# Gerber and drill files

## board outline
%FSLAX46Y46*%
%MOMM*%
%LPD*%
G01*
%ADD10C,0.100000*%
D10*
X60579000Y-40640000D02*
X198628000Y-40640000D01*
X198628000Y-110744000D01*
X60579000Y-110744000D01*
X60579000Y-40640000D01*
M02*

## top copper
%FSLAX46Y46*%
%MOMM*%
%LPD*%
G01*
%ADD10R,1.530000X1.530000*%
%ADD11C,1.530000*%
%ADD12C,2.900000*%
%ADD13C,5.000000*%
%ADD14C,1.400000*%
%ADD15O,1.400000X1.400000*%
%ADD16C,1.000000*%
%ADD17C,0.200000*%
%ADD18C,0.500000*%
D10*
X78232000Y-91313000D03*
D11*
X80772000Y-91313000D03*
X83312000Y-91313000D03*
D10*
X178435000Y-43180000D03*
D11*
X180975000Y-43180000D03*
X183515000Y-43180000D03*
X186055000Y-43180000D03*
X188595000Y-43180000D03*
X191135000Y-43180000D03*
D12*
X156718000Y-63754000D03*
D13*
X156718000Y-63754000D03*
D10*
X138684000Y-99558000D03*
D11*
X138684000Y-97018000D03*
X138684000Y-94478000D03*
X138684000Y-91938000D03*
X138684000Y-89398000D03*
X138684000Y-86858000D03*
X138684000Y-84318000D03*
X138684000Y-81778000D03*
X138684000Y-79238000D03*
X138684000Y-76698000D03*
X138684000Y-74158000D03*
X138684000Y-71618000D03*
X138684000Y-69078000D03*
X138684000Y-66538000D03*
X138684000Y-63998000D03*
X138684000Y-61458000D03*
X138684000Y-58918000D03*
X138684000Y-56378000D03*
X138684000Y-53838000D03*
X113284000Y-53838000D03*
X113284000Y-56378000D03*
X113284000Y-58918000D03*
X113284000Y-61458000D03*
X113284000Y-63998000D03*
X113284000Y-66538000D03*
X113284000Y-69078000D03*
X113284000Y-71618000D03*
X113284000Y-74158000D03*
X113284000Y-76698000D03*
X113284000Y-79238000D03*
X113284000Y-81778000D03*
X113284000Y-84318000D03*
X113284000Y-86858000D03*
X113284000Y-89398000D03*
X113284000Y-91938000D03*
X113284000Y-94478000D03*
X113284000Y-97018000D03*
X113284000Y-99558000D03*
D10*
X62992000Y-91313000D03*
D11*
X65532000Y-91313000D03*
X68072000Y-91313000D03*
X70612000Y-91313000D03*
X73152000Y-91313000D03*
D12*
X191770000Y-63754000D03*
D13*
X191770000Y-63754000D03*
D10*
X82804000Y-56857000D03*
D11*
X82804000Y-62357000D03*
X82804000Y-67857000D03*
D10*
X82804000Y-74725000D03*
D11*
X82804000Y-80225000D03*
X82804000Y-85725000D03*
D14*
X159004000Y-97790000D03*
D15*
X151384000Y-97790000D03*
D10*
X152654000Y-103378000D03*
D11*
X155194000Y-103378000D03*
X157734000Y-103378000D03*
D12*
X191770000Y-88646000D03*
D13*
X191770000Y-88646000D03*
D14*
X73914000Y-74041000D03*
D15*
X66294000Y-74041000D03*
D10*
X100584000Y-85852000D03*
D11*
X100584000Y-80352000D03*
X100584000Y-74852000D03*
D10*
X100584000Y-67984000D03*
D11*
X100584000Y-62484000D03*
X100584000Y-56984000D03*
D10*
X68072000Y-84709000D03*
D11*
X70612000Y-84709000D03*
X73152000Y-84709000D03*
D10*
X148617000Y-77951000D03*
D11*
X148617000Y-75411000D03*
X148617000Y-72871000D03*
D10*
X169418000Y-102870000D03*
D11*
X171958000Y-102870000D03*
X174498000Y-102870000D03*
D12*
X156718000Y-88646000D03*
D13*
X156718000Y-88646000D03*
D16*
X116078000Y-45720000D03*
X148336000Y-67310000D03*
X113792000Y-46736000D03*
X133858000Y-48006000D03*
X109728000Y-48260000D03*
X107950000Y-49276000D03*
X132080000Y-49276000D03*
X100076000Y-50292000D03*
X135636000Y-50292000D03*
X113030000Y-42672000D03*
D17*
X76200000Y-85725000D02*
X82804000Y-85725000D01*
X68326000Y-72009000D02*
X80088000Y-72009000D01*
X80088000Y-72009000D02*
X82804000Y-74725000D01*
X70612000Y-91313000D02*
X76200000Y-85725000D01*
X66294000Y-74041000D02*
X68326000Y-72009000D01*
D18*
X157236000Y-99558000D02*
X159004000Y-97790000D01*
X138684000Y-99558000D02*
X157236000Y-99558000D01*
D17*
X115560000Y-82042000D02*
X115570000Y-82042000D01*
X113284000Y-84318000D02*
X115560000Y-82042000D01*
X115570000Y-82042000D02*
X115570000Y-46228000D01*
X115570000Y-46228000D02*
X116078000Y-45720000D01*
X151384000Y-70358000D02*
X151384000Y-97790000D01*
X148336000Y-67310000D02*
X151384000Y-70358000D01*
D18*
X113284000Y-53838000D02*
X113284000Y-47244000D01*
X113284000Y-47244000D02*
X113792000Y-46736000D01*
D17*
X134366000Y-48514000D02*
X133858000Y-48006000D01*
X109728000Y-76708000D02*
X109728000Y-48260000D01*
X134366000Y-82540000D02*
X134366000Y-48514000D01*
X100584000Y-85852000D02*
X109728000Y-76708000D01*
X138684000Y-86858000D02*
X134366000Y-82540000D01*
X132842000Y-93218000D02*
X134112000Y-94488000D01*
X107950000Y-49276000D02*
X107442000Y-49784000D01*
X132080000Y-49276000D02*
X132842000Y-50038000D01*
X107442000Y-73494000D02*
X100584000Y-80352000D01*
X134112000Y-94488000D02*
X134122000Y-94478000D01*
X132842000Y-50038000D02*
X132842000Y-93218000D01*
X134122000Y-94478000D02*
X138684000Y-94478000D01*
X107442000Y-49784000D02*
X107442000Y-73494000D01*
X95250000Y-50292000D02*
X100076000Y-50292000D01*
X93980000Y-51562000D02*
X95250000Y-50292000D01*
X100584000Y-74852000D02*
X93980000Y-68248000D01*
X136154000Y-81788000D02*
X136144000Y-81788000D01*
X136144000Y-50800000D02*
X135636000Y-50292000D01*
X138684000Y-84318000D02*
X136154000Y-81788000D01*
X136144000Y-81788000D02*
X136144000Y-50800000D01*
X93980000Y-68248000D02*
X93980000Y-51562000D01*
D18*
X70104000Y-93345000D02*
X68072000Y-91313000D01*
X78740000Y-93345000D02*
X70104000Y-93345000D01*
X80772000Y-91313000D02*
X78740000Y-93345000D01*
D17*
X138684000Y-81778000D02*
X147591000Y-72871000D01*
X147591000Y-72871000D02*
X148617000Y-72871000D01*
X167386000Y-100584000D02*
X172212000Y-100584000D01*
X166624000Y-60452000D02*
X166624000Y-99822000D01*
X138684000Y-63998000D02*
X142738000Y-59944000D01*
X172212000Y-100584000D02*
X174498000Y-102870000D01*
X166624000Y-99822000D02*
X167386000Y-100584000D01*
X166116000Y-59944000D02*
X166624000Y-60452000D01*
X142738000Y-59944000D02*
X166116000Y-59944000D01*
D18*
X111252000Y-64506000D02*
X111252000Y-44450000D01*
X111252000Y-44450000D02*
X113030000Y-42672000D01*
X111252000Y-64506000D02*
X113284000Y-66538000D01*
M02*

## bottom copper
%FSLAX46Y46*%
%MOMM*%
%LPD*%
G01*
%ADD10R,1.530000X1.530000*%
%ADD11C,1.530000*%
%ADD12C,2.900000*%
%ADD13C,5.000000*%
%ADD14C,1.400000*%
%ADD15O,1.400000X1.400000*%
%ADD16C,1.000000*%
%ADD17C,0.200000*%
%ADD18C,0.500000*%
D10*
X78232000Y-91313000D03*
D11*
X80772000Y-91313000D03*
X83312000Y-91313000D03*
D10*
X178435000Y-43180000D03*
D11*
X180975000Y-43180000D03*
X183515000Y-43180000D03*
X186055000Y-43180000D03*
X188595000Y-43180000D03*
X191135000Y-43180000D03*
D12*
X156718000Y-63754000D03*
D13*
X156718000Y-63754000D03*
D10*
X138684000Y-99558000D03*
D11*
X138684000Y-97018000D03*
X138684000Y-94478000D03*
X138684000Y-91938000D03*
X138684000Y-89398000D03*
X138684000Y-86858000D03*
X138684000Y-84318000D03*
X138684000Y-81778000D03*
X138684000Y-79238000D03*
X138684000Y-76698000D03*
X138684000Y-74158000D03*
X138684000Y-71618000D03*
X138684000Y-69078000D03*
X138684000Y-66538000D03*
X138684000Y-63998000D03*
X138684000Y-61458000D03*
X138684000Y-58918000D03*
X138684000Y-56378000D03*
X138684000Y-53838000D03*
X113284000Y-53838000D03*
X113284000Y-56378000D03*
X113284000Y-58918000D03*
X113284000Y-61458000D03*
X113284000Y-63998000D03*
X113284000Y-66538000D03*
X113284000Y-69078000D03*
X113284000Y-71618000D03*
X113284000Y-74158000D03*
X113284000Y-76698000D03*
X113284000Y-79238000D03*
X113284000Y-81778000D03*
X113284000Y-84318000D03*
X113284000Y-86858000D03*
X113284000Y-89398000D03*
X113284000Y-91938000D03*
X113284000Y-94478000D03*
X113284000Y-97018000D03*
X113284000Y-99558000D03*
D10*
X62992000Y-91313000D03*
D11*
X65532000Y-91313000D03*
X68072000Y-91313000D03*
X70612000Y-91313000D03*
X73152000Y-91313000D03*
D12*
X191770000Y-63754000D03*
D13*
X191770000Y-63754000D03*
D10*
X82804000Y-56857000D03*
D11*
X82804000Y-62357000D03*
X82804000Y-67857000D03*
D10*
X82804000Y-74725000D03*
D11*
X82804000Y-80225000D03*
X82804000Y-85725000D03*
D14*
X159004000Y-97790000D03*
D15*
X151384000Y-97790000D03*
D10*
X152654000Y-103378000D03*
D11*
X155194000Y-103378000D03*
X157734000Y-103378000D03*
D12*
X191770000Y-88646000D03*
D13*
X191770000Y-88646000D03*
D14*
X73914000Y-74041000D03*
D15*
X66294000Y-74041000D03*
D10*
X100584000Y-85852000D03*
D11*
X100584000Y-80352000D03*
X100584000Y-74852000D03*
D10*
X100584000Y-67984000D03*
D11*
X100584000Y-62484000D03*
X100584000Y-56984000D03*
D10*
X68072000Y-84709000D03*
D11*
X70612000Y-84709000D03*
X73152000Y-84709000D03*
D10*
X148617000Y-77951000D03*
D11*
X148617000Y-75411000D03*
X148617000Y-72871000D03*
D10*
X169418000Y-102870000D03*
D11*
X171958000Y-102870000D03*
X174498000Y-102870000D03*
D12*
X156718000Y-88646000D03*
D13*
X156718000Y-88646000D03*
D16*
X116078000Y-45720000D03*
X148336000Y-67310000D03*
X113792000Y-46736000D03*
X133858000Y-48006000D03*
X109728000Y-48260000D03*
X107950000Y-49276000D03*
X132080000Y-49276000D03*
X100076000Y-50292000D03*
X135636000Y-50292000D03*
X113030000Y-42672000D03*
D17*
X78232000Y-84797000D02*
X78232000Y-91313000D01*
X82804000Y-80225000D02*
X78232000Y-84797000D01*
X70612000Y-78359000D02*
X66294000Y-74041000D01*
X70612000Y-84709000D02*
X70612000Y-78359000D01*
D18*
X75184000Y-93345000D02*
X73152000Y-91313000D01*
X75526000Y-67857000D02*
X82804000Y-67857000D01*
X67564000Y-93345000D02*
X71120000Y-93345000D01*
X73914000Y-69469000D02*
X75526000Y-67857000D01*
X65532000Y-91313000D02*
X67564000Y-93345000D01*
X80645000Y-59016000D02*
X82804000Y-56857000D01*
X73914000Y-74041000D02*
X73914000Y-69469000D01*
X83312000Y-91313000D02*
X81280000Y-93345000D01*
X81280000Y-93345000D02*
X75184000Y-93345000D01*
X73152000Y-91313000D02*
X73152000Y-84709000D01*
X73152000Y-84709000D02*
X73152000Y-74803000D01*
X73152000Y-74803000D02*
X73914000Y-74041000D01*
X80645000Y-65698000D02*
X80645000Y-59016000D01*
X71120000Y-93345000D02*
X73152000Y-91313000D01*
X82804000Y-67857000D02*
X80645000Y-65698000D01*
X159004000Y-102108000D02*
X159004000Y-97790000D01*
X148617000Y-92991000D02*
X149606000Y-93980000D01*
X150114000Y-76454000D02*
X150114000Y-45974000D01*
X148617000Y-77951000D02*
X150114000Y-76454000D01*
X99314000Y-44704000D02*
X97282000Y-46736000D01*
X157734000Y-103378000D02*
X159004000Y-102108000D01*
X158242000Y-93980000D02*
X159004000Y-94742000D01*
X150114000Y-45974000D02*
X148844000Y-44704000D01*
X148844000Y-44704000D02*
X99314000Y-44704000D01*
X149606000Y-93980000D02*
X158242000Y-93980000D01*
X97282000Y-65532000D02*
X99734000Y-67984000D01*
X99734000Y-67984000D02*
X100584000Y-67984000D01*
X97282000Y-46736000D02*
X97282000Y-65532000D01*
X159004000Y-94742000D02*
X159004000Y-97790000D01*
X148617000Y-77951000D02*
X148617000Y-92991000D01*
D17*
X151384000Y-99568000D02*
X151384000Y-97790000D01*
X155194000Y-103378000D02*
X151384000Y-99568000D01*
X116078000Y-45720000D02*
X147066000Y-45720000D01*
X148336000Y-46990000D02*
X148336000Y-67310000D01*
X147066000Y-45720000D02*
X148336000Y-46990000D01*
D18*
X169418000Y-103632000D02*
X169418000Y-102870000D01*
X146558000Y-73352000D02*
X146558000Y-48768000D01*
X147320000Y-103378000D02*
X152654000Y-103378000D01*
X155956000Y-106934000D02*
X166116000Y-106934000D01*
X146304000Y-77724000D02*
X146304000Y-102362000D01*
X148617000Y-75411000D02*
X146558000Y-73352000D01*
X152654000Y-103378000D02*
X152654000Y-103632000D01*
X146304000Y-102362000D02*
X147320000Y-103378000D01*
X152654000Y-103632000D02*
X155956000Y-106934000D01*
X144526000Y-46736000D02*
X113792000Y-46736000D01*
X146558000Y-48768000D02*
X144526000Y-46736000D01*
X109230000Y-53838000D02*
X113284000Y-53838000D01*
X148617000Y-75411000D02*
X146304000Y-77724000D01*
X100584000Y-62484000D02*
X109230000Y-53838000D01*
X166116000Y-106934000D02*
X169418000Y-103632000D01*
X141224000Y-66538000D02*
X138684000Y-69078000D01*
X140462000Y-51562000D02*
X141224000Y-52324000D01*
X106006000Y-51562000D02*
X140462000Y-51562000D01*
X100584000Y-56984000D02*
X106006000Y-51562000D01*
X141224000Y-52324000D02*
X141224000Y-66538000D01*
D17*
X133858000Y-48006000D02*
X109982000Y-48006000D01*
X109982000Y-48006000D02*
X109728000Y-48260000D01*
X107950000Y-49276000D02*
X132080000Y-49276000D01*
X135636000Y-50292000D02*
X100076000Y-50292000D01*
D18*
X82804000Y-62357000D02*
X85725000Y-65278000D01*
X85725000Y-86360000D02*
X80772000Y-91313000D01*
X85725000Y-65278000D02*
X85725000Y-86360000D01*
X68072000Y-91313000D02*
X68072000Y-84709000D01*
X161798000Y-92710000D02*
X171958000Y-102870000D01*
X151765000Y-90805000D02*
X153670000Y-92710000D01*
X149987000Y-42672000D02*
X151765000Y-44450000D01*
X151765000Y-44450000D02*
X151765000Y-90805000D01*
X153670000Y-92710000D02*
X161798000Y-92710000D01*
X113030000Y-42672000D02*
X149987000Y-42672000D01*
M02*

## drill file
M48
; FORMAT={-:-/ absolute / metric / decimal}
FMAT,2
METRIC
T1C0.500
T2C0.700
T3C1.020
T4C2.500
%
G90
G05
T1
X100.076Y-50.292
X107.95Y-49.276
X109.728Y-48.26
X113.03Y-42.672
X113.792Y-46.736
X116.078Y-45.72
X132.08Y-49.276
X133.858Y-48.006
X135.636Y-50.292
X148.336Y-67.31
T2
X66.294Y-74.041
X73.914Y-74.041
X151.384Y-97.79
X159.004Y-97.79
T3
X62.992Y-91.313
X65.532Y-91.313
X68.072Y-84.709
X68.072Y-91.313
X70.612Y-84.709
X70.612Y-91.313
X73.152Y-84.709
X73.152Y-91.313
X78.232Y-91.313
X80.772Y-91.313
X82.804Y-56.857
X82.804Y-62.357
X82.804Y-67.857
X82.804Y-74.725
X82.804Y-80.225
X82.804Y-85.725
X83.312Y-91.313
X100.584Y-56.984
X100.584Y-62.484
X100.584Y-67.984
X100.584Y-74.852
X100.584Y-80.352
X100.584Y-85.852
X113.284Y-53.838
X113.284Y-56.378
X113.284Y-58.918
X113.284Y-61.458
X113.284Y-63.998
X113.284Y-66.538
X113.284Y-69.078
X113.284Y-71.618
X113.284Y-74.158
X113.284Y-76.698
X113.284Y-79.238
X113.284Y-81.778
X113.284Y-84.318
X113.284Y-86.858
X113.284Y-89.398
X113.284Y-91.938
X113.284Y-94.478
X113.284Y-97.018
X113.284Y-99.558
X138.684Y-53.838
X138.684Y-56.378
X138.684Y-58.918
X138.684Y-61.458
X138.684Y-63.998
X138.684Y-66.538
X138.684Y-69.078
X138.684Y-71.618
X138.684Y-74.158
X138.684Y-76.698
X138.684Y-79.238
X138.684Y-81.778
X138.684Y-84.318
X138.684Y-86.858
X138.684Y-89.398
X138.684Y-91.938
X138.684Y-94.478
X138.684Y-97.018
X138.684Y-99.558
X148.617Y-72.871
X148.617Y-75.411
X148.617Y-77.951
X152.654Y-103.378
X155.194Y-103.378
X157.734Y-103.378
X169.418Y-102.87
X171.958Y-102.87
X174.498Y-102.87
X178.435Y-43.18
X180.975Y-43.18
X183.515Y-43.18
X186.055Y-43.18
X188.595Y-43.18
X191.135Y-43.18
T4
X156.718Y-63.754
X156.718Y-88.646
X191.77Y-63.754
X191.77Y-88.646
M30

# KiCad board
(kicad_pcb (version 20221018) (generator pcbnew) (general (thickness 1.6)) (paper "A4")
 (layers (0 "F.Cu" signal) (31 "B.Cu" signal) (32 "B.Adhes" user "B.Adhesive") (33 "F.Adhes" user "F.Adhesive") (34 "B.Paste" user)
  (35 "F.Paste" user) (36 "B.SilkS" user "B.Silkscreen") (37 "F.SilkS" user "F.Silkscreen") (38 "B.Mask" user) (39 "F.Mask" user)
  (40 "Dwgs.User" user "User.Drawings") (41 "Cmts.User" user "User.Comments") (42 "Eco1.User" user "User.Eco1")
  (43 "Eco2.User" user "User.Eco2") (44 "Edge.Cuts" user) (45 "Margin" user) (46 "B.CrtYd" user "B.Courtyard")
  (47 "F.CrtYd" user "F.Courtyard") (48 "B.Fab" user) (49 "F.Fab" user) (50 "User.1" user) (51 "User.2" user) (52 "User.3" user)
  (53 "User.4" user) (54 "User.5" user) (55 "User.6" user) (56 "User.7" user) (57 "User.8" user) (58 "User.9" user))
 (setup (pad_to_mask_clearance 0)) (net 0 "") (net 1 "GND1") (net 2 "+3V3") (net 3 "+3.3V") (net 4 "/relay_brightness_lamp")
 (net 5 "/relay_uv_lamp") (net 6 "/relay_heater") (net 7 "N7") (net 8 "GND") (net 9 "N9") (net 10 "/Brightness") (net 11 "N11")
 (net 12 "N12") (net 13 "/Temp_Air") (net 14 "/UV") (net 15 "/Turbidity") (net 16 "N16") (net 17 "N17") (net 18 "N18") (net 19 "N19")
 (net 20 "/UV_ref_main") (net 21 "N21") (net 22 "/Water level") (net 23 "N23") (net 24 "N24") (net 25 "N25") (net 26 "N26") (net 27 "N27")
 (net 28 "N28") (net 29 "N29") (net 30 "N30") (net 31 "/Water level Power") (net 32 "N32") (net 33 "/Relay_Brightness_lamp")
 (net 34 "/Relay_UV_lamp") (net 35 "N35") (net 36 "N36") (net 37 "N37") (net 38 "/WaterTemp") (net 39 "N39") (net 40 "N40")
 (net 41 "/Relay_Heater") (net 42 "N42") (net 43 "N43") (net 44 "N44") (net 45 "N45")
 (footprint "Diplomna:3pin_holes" (layer "F.Cu") (at 85.852 93.853)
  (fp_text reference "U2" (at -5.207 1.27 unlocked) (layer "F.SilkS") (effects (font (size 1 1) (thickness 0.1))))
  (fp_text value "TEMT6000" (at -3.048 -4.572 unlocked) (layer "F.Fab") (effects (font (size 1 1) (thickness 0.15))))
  (pad "1" thru_hole rect (at -7.62 -2.54) (size 1.53 1.53) (drill 1.02) (layers "*.Cu" "*.Mask") (solder_mask_margin 0.102))
  (pad "2" thru_hole circle (at -5.08 -2.54) (size 1.53 1.53) (drill 1.02) (layers "*.Cu" "*.Mask") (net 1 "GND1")
   (solder_mask_margin 0.102))
  (pad "3" thru_hole circle (at -2.54 -2.54) (size 1.53 1.53) (drill 1.02) (layers "*.Cu" "*.Mask") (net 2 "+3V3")
   (solder_mask_margin 0.102)))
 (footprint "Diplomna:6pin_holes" (layer "F.Cu") (at 193.675 48.895)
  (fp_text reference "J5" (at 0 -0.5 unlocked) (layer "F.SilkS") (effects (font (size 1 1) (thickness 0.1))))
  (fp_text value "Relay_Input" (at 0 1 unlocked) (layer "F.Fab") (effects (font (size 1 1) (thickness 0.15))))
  (pad "1" thru_hole rect (at -15.24 -5.715) (size 1.53 1.53) (drill 1.02) (layers "*.Cu" "*.Mask") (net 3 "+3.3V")
   (solder_mask_margin 0.102))
  (pad "2" thru_hole circle (at -12.7 -5.715) (size 1.53 1.53) (drill 1.02) (layers "*.Cu" "*.Mask") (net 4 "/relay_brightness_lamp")
   (solder_mask_margin 0.102))
  (pad "3" thru_hole circle (at -10.16 -5.715) (size 1.53 1.53) (drill 1.02) (layers "*.Cu" "*.Mask") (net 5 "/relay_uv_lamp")
   (solder_mask_margin 0.102))
  (pad "4" thru_hole circle (at -7.62 -5.715) (size 1.53 1.53) (drill 1.02) (layers "*.Cu" "*.Mask") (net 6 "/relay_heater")
   (solder_mask_margin 0.102))
  (pad "5" thru_hole circle (at -5.08 -5.715) (size 1.53 1.53) (drill 1.02) (layers "*.Cu" "*.Mask") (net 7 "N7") (solder_mask_margin 0.102))
  (pad "6" thru_hole circle (at -2.54 -5.715) (size 1.53 1.53) (drill 1.02) (layers "*.Cu" "*.Mask") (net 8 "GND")
   (solder_mask_margin 0.102)))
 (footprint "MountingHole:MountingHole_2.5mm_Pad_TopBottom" (layer "F.Cu") (at 156.718 63.754)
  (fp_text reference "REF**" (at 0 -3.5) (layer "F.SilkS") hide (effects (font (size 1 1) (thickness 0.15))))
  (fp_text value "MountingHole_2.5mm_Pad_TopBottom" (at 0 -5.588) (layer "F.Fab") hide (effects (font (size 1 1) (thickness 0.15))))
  (pad "1" thru_hole circle (at 0 0) (size 2.9 2.9) (drill 2.5) (layers "*.Cu" "*.Mask"))
  (pad "1" connect circle (at 0 0) (size 5 5) (layers "F.Cu" "F.Mask"))
  (pad "1" connect circle (at 0 0) (size 5 5) (layers "B.Cu" "B.Mask")))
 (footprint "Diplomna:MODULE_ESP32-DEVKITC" (layer "F.Cu") (at 125.984 76.708 180)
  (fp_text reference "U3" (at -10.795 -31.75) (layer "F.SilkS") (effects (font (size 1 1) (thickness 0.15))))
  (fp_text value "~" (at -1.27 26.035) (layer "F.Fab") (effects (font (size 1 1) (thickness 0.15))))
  (pad "1" thru_hole rect (at -12.7 -22.85 180) (size 1.53 1.53) (drill 1.02) (layers "*.Cu" "*.Mask") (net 3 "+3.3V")
   (solder_mask_margin 0.102))
  (pad "2" thru_hole circle (at -12.7 -20.31 180) (size 1.53 1.53) (drill 1.02) (layers "*.Cu" "*.Mask") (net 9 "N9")
   (solder_mask_margin 0.102))
  (pad "3" thru_hole circle (at -12.7 -17.77 180) (size 1.53 1.53) (drill 1.02) (layers "*.Cu" "*.Mask") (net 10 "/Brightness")
   (solder_mask_margin 0.102))
  (pad "4" thru_hole circle (at -12.7 -15.23 180) (size 1.53 1.53) (drill 1.02) (layers "*.Cu" "*.Mask") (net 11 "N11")
   (solder_mask_margin 0.102))
  (pad "5" thru_hole circle (at -12.7 -12.69 180) (size 1.53 1.53) (drill 1.02) (layers "*.Cu" "*.Mask") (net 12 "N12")
   (solder_mask_margin 0.102))
  (pad "6" thru_hole circle (at -12.7 -10.15 180) (size 1.53 1.53) (drill 1.02) (layers "*.Cu" "*.Mask") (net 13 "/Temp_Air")
   (solder_mask_margin 0.102))
  (pad "7" thru_hole circle (at -12.7 -7.61 180) (size 1.53 1.53) (drill 1.02) (layers "*.Cu" "*.Mask") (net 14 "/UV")
   (solder_mask_margin 0.102))
  (pad "8" thru_hole circle (at -12.7 -5.07 180) (size 1.53 1.53) (drill 1.02) (layers "*.Cu" "*.Mask") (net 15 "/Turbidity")
   (solder_mask_margin 0.102))
  (pad "9" thru_hole circle (at -12.7 -2.53 180) (size 1.53 1.53) (drill 1.02) (layers "*.Cu" "*.Mask") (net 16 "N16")
   (solder_mask_margin 0.102))
  (pad "10" thru_hole circle (at -12.7 0.01 180) (size 1.53 1.53) (drill 1.02) (layers "*.Cu" "*.Mask") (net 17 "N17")
   (solder_mask_margin 0.102))
  (pad "11" thru_hole circle (at -12.7 2.55 180) (size 1.53 1.53) (drill 1.02) (layers "*.Cu" "*.Mask") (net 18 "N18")
   (solder_mask_margin 0.102))
  (pad "12" thru_hole circle (at -12.7 5.09 180) (size 1.53 1.53) (drill 1.02) (layers "*.Cu" "*.Mask") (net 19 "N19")
   (solder_mask_margin 0.102))
  (pad "13" thru_hole circle (at -12.7 7.63 180) (size 1.53 1.53) (drill 1.02) (layers "*.Cu" "*.Mask") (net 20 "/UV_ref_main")
   (solder_mask_margin 0.102))
  (pad "14" thru_hole circle (at -12.7 10.17 180) (size 1.53 1.53) (drill 1.02) (layers "*.Cu" "*.Mask") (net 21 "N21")
   (solder_mask_margin 0.102))
  (pad "15" thru_hole circle (at -12.7 12.71 180) (size 1.53 1.53) (drill 1.02) (layers "*.Cu" "*.Mask") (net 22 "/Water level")
   (solder_mask_margin 0.102))
  (pad "16" thru_hole circle (at -12.7 15.25 180) (size 1.53 1.53) (drill 1.02) (layers "*.Cu" "*.Mask") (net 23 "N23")
   (solder_mask_margin 0.102))
  (pad "17" thru_hole circle (at -12.7 17.79 180) (size 1.53 1.53) (drill 1.02) (layers "*.Cu" "*.Mask") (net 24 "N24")
   (solder_mask_margin 0.102))
  (pad "18" thru_hole circle (at -12.7 20.33 180) (size 1.53 1.53) (drill 1.02) (layers "*.Cu" "*.Mask") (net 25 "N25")
   (solder_mask_margin 0.102))
  (pad "19" thru_hole circle (at -12.7 22.87 180) (size 1.53 1.53) (drill 1.02) (layers "*.Cu" "*.Mask") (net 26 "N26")
   (solder_mask_margin 0.102))
  (pad "20" thru_hole circle (at 12.7 22.87 180) (size 1.53 1.53) (drill 1.02) (layers "*.Cu" "*.Mask") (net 8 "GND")
   (solder_mask_margin 0.102))
  (pad "21" thru_hole circle (at 12.7 20.33 180) (size 1.53 1.53) (drill 1.02) (layers "*.Cu" "*.Mask") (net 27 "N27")
   (solder_mask_margin 0.102))
  (pad "22" thru_hole circle (at 12.7 17.79 180) (size 1.53 1.53) (drill 1.02) (layers "*.Cu" "*.Mask") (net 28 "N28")
   (solder_mask_margin 0.102))
  (pad "23" thru_hole circle (at 12.7 15.25 180) (size 1.53 1.53) (drill 1.02) (layers "*.Cu" "*.Mask") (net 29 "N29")
   (solder_mask_margin 0.102))
  (pad "24" thru_hole circle (at 12.7 12.71 180) (size 1.53 1.53) (drill 1.02) (layers "*.Cu" "*.Mask") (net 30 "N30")
   (solder_mask_margin 0.102))
  (pad "25" thru_hole circle (at 12.7 10.17 180) (size 1.53 1.53) (drill 1.02) (layers "*.Cu" "*.Mask") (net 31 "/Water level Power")
   (solder_mask_margin 0.102))
  (pad "26" thru_hole circle (at 12.7 7.63 180) (size 1.53 1.53) (drill 1.02) (layers "*.Cu" "*.Mask") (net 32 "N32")
   (solder_mask_margin 0.102))
  (pad "27" thru_hole circle (at 12.7 5.09 180) (size 1.53 1.53) (drill 1.02) (layers "*.Cu" "*.Mask") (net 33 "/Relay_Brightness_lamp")
   (solder_mask_margin 0.102))
  (pad "28" thru_hole circle (at 12.7 2.55 180) (size 1.53 1.53) (drill 1.02) (layers "*.Cu" "*.Mask") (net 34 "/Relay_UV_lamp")
   (solder_mask_margin 0.102))
  (pad "29" thru_hole circle (at 12.7 0.01 180) (size 1.53 1.53) (drill 1.02) (layers "*.Cu" "*.Mask") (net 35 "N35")
   (solder_mask_margin 0.102))
  (pad "30" thru_hole circle (at 12.7 -2.53 180) (size 1.53 1.53) (drill 1.02) (layers "*.Cu" "*.Mask") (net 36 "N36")
   (solder_mask_margin 0.102))
  (pad "31" thru_hole circle (at 12.7 -5.07 180) (size 1.53 1.53) (drill 1.02) (layers "*.Cu" "*.Mask") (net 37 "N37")
   (solder_mask_margin 0.102))
  (pad "32" thru_hole circle (at 12.7 -7.61 180) (size 1.53 1.53) (drill 1.02) (layers "*.Cu" "*.Mask") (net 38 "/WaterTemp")
   (solder_mask_margin 0.102))
  (pad "33" thru_hole circle (at 12.7 -10.15 180) (size 1.53 1.53) (drill 1.02) (layers "*.Cu" "*.Mask") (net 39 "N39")
   (solder_mask_margin 0.102))
  (pad "34" thru_hole circle (at 12.7 -12.69 180) (size 1.53 1.53) (drill 1.02) (layers "*.Cu" "*.Mask") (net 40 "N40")
   (solder_mask_margin 0.102))
  (pad "35" thru_hole circle (at 12.7 -15.23 180) (size 1.53 1.53) (drill 1.02) (layers "*.Cu" "*.Mask") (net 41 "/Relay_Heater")
   (solder_mask_margin 0.102))
  (pad "36" thru_hole circle (at 12.7 -17.77 180) (size 1.53 1.53) (drill 1.02) (layers "*.Cu" "*.Mask") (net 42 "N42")
   (solder_mask_margin 0.102))
  (pad "37" thru_hole circle (at 12.7 -20.31 180) (size 1.53 1.53) (drill 1.02) (layers "*.Cu" "*.Mask") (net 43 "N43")
   (solder_mask_margin 0.102))
  (pad "38" thru_hole circle (at 12.7 -22.85 180) (size 1.53 1.53) (drill 1.02) (layers "*.Cu" "*.Mask") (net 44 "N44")
   (solder_mask_margin 0.102)))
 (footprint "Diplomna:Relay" (layer "F.Cu") (at 254.508 101.092 -90)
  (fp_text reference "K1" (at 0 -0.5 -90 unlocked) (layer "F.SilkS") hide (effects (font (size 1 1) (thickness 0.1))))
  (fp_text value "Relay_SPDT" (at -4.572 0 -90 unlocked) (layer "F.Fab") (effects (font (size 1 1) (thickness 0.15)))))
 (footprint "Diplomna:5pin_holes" (layer "F.Cu") (at 78.232 97.028)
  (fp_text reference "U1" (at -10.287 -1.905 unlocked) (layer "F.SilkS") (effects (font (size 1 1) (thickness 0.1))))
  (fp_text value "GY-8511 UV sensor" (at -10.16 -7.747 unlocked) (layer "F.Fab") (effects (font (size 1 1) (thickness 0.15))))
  (pad "1" thru_hole rect (at -15.24 -5.715) (size 1.53 1.53) (drill 1.02) (layers "*.Cu" "*.Mask") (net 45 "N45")
   (solder_mask_margin 0.102))
  (pad "2" thru_hole circle (at -12.7 -5.715) (size 1.53 1.53) (drill 1.02) (layers "*.Cu" "*.Mask") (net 2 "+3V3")
   (solder_mask_margin 0.102))
  (pad "3" thru_hole circle (at -10.16 -5.715) (size 1.53 1.53) (drill 1.02) (layers "*.Cu" "*.Mask") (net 1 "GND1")
   (solder_mask_margin 0.102))
  (pad "4" thru_hole circle (at -7.62 -5.715) (size 1.53 1.53) (drill 1.02) (layers "*.Cu" "*.Mask") (solder_mask_margin 0.102))
  (pad "5" thru_hole circle (at -5.08 -5.715) (size 1.53 1.53) (drill 1.02) (layers "*.Cu" "*.Mask") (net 2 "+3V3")
   (solder_mask_margin 0.102)))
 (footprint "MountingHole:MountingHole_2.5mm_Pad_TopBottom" (layer "F.Cu") (at 191.77 63.754)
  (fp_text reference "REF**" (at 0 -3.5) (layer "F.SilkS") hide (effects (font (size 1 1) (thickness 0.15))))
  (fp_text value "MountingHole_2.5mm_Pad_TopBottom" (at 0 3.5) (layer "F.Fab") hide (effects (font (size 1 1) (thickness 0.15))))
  (pad "1" thru_hole circle (at 0 0) (size 2.9 2.9) (drill 2.5) (layers "*.Cu" "*.Mask"))
  (pad "1" connect circle (at 0 0) (size 5 5) (layers "F.Cu" "F.Mask"))
  (pad "1" connect circle (at 0 0) (size 5 5) (layers "B.Cu" "B.Mask")))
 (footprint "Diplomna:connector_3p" (layer "F.Cu") (at 82.804 62.357 -90)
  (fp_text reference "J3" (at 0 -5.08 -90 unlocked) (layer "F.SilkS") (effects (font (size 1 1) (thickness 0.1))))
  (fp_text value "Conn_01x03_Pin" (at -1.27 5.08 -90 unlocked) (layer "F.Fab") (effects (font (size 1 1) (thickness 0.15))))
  (pad "1" thru_hole rect (at -5.5 0 270) (size 1.53 1.53) (drill 1.02) (layers "*.Cu" "*.Mask") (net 2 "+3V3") (solder_mask_margin 0.102))
  (pad "2" thru_hole circle (at 0 0 270) (size 1.53 1.53) (drill 1.02) (layers "*.Cu" "*.Mask") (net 1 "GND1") (solder_mask_margin 0.102))
  (pad "3" thru_hole circle (at 5.5 0 270) (size 1.53 1.53) (drill 1.02) (layers "*.Cu" "*.Mask") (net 2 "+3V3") (solder_mask_margin 0.102)))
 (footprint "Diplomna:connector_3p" (layer "F.Cu") (at 82.804 80.225 -90)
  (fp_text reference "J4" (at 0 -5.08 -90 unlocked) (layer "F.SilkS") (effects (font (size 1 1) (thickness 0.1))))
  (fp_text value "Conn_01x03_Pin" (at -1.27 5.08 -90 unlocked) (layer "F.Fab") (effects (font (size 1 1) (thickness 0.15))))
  (pad "1" thru_hole rect (at -5.5 0 270) (size 1.53 1.53) (drill 1.02) (layers "*.Cu" "*.Mask") (solder_mask_margin 0.102))
  (pad "2" thru_hole circle (at 0 0 270) (size 1.53 1.53) (drill 1.02) (layers "*.Cu" "*.Mask") (solder_mask_margin 0.102))
  (pad "3" thru_hole circle (at 5.5 0 270) (size 1.53 1.53) (drill 1.02) (layers "*.Cu" "*.Mask") (solder_mask_margin 0.102)))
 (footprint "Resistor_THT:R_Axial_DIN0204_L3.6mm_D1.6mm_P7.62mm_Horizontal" (layer "F.Cu") (at 159.004 97.79 180)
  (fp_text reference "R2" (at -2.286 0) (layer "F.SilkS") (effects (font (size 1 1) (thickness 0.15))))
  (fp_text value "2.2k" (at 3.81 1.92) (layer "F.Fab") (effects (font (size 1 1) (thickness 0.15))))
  (pad "1" thru_hole circle (at 0 0 180) (size 1.4 1.4) (drill 0.7) (layers "*.Cu" "*.Mask") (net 3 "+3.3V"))
  (pad "2" thru_hole oval (at 7.62 0 180) (size 1.4 1.4) (drill 0.7) (layers "*.Cu" "*.Mask") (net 38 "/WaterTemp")))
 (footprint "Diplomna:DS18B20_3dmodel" (layer "F.Cu") (at 160.274 105.918)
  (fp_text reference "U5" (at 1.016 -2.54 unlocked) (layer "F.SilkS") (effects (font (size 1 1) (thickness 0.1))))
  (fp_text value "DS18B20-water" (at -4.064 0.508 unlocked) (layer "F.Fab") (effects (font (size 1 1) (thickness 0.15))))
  (pad "1" thru_hole rect (at -7.62 -2.54) (size 1.53 1.53) (drill 1.02) (layers "*.Cu" "*.Mask") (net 8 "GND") (solder_mask_margin 0.102))
  (pad "2" thru_hole circle (at -5.08 -2.54) (size 1.53 1.53) (drill 1.02) (layers "*.Cu" "*.Mask") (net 38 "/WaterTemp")
   (solder_mask_margin 0.102))
  (pad "3" thru_hole circle (at -2.54 -2.54) (size 1.53 1.53) (drill 1.02) (layers "*.Cu" "*.Mask") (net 3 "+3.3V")
   (solder_mask_margin 0.102)))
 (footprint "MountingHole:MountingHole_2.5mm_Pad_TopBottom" (layer "F.Cu") (at 191.77 88.646)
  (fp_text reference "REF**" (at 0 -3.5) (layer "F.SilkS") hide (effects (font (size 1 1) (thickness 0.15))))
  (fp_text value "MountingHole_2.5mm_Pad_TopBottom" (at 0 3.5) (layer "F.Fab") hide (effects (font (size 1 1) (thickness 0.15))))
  (pad "1" thru_hole circle (at 0 0) (size 2.9 2.9) (drill 2.5) (layers "*.Cu" "*.Mask"))
  (pad "1" connect circle (at 0 0) (size 5 5) (layers "F.Cu" "F.Mask"))
  (pad "1" connect circle (at 0 0) (size 5 5) (layers "B.Cu" "B.Mask")))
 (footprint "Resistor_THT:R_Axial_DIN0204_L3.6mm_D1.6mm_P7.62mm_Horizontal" (layer "F.Cu") (at 73.914 74.041 180)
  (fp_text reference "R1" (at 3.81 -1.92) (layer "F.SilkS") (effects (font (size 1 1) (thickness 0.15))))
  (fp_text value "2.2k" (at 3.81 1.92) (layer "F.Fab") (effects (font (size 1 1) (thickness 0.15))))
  (pad "1" thru_hole circle (at 0 0 180) (size 1.4 1.4) (drill 0.7) (layers "*.Cu" "*.Mask") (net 2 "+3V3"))
  (pad "2" thru_hole oval (at 7.62 0 180) (size 1.4 1.4) (drill 0.7) (layers "*.Cu" "*.Mask")))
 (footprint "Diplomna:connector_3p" (layer "F.Cu") (at 100.584 80.352 90)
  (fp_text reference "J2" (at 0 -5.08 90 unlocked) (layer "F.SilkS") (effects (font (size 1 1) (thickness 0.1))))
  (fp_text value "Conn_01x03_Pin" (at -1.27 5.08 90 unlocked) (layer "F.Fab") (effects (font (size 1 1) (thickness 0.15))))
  (pad "1" thru_hole rect (at -5.5 0 90) (size 1.53 1.53) (drill 1.02) (layers "*.Cu" "*.Mask") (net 13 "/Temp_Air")
   (solder_mask_margin 0.102))
  (pad "2" thru_hole circle (at 0 0 90) (size 1.53 1.53) (drill 1.02) (layers "*.Cu" "*.Mask") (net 10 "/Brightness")
   (solder_mask_margin 0.102))
  (pad "3" thru_hole circle (at 5.5 0 90) (size 1.53 1.53) (drill 1.02) (layers "*.Cu" "*.Mask") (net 14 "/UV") (solder_mask_margin 0.102)))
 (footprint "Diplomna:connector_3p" (layer "F.Cu") (at 100.584 62.484 90)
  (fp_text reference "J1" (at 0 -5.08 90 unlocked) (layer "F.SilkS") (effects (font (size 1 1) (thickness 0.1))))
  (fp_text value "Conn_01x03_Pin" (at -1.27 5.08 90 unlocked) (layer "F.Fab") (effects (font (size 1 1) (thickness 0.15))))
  (pad "1" thru_hole rect (at -5.5 0 90) (size 1.53 1.53) (drill 1.02) (layers "*.Cu" "*.Mask") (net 3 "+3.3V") (solder_mask_margin 0.102))
  (pad "2" thru_hole circle (at 0 0 90) (size 1.53 1.53) (drill 1.02) (layers "*.Cu" "*.Mask") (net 8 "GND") (solder_mask_margin 0.102))
  (pad "3" thru_hole circle (at 5.5 0 90) (size 1.53 1.53) (drill 1.02) (layers "*.Cu" "*.Mask") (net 20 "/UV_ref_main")
   (solder_mask_margin 0.102)))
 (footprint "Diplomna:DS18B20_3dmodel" (layer "F.Cu") (at 75.692 87.249)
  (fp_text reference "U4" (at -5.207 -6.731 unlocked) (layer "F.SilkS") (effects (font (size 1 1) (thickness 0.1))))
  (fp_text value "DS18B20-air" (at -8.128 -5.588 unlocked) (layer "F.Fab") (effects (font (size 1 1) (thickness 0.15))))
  (pad "1" thru_hole rect (at -7.62 -2.54) (size 1.53 1.53) (drill 1.02) (layers "*.Cu" "*.Mask") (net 1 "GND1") (solder_mask_margin 0.102))
  (pad "2" thru_hole circle (at -5.08 -2.54) (size 1.53 1.53) (drill 1.02) (layers "*.Cu" "*.Mask") (solder_mask_margin 0.102))
  (pad "3" thru_hole circle (at -2.54 -2.54) (size 1.53 1.53) (drill 1.02) (layers "*.Cu" "*.Mask") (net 2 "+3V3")
   (solder_mask_margin 0.102)))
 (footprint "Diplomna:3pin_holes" (layer "F.Cu") (at 151.157 70.331 90)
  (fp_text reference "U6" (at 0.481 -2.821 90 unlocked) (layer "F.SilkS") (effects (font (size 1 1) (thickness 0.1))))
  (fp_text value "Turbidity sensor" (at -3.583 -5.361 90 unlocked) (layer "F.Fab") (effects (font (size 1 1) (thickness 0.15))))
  (pad "1" thru_hole rect (at -7.62 -2.54 90) (size 1.53 1.53) (drill 1.02) (layers "*.Cu" "*.Mask") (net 3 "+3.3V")
   (solder_mask_margin 0.102))
  (pad "2" thru_hole circle (at -5.08 -2.54 90) (size 1.53 1.53) (drill 1.02) (layers "*.Cu" "*.Mask") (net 8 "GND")
   (solder_mask_margin 0.102))
  (pad "3" thru_hole circle (at -2.54 -2.54 90) (size 1.53 1.53) (drill 1.02) (layers "*.Cu" "*.Mask") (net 15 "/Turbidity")
   (solder_mask_margin 0.102)))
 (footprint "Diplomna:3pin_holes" (layer "F.Cu") (at 177.038 105.41)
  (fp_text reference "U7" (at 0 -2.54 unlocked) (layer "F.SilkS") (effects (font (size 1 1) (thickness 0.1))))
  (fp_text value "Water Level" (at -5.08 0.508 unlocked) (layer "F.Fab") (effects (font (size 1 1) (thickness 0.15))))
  (pad "1" thru_hole rect (at -7.62 -2.54) (size 1.53 1.53) (drill 1.02) (layers "*.Cu" "*.Mask") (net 8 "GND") (solder_mask_margin 0.102))
  (pad "2" thru_hole circle (at -5.08 -2.54) (size 1.53 1.53) (drill 1.02) (layers "*.Cu" "*.Mask") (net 31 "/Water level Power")
   (solder_mask_margin 0.102))
  (pad "3" thru_hole circle (at -2.54 -2.54) (size 1.53 1.53) (drill 1.02) (layers "*.Cu" "*.Mask") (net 22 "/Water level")
   (solder_mask_margin 0.102)))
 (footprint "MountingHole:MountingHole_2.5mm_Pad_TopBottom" (layer "F.Cu") (at 156.718 88.646)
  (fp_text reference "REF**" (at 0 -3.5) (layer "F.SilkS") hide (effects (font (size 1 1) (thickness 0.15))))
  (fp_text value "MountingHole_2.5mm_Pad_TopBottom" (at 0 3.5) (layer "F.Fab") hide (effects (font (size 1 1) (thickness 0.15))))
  (pad "1" thru_hole circle (at 0 0) (size 2.9 2.9) (drill 2.5) (layers "*.Cu" "*.Mask"))
  (pad "1" connect circle (at 0 0) (size 5 5) (layers "F.Cu" "F.Mask"))
  (pad "1" connect circle (at 0 0) (size 5 5) (layers "B.Cu" "B.Mask")))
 (gr_rect (start 60.579 40.64) (end 198.628 110.744) (stroke (width 0.1) (type default)) (fill none) (layer "Edge.Cuts"))
 (segment (start 76.2 85.725) (end 82.804 85.725) (width 0.2) (layer "F.Cu") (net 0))
 (segment (start 68.326 72.009) (end 80.088 72.009) (width 0.2) (layer "F.Cu") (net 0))
 (segment (start 80.088 72.009) (end 82.804 74.725) (width 0.2) (layer "F.Cu") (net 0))
 (segment (start 70.612 91.313) (end 76.2 85.725) (width 0.2) (layer "F.Cu") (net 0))
 (segment (start 66.294 74.041) (end 68.326 72.009) (width 0.2) (layer "F.Cu") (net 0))
 (segment (start 78.232 84.797) (end 78.232 91.313) (width 0.2) (layer "B.Cu") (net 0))
 (segment (start 82.804 80.225) (end 78.232 84.797) (width 0.2) (layer "B.Cu") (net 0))
 (segment (start 70.612 78.359) (end 66.294 74.041) (width 0.2) (layer "B.Cu") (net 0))
 (segment (start 70.612 84.709) (end 70.612 78.359) (width 0.2) (layer "B.Cu") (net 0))
 (segment (start 75.184 93.345) (end 73.152 91.313) (width 0.5) (layer "B.Cu") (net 2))
 (segment (start 75.526 67.857) (end 82.804 67.857) (width 0.5) (layer "B.Cu") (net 2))
 (segment (start 67.564 93.345) (end 71.12 93.345) (width 0.5) (layer "B.Cu") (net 2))
 (segment (start 73.914 69.469) (end 75.526 67.857) (width 0.5) (layer "B.Cu") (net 2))
 (segment (start 65.532 91.313) (end 67.564 93.345) (width 0.5) (layer "B.Cu") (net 2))
 (segment (start 80.645 59.016) (end 82.804 56.857) (width 0.5) (layer "B.Cu") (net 2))
 (segment (start 73.914 74.041) (end 73.914 69.469) (width 0.5) (layer "B.Cu") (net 2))
 (segment (start 83.312 91.313) (end 81.28 93.345) (width 0.5) (layer "B.Cu") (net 2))
 (segment (start 81.28 93.345) (end 75.184 93.345) (width 0.5) (layer "B.Cu") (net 2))
 (segment (start 73.152 91.313) (end 73.152 84.709) (width 0.5) (layer "B.Cu") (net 2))
 (segment (start 73.152 84.709) (end 73.152 74.803) (width 0.5) (layer "B.Cu") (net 2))
 (segment (start 73.152 74.803) (end 73.914 74.041) (width 0.5) (layer "B.Cu") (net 2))
 (segment (start 80.645 65.698) (end 80.645 59.016) (width 0.5) (layer "B.Cu") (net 2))
 (segment (start 71.12 93.345) (end 73.152 91.313) (width 0.5) (layer "B.Cu") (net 2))
 (segment (start 82.804 67.857) (end 80.645 65.698) (width 0.5) (layer "B.Cu") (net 2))
 (segment (start 157.236 99.558) (end 159.004 97.79) (width 0.5) (layer "F.Cu") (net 3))
 (segment (start 138.684 99.558) (end 157.236 99.558) (width 0.5) (layer "F.Cu") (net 3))
 (segment (start 159.004 102.108) (end 159.004 97.79) (width 0.5) (layer "B.Cu") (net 3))
 (segment (start 148.617 92.991) (end 149.606 93.98) (width 0.5) (layer "B.Cu") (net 3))
 (segment (start 150.114 76.454) (end 150.114 45.974) (width 0.5) (layer "B.Cu") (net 3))
 (segment (start 148.617 77.951) (end 150.114 76.454) (width 0.5) (layer "B.Cu") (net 3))
 (segment (start 99.314 44.704) (end 97.282 46.736) (width 0.5) (layer "B.Cu") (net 3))
 (segment (start 157.734 103.378) (end 159.004 102.108) (width 0.5) (layer "B.Cu") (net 3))
 (segment (start 158.242 93.98) (end 159.004 94.742) (width 0.5) (layer "B.Cu") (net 3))
 (segment (start 150.114 45.974) (end 148.844 44.704) (width 0.5) (layer "B.Cu") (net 3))
 (segment (start 148.844 44.704) (end 99.314 44.704) (width 0.5) (layer "B.Cu") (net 3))
 (segment (start 149.606 93.98) (end 158.242 93.98) (width 0.5) (layer "B.Cu") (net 3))
 (segment (start 97.282 65.532) (end 99.734 67.984) (width 0.5) (layer "B.Cu") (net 3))
 (segment (start 99.734 67.984) (end 100.584 67.984) (width 0.5) (layer "B.Cu") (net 3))
 (segment (start 97.282 46.736) (end 97.282 65.532) (width 0.5) (layer "B.Cu") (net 3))
 (segment (start 159.004 94.742) (end 159.004 97.79) (width 0.5) (layer "B.Cu") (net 3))
 (segment (start 148.617 77.951) (end 148.617 92.991) (width 0.5) (layer "B.Cu") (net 3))
 (segment (start 115.56 82.042) (end 115.57 82.042) (width 0.2) (layer "F.Cu") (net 38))
 (segment (start 113.284 84.318) (end 115.56 82.042) (width 0.2) (layer "F.Cu") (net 38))
 (segment (start 115.57 82.042) (end 115.57 46.228) (width 0.2) (layer "F.Cu") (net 38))
 (segment (start 115.57 46.228) (end 116.078 45.72) (width 0.2) (layer "F.Cu") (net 38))
 (segment (start 151.384 70.358) (end 151.384 97.79) (width 0.2) (layer "F.Cu") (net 38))
 (segment (start 148.336 67.31) (end 151.384 70.358) (width 0.2) (layer "F.Cu") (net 38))
 (via (at 116.078 45.72) (size 1) (drill 0.5) (layers "F.Cu" "B.Cu") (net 38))
 (via (at 148.336 67.31) (size 1) (drill 0.5) (layers "F.Cu" "B.Cu") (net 38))
 (segment (start 151.384 99.568) (end 151.384 97.79) (width 0.2) (layer "B.Cu") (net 38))
 (segment (start 155.194 103.378) (end 151.384 99.568) (width 0.2) (layer "B.Cu") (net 38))
 (segment (start 116.078 45.72) (end 147.066 45.72) (width 0.2) (layer "B.Cu") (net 38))
 (segment (start 148.336 46.99) (end 148.336 67.31) (width 0.2) (layer "B.Cu") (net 38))
 (segment (start 147.066 45.72) (end 148.336 46.99) (width 0.2) (layer "B.Cu") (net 38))
 (segment (start 113.284 53.838) (end 113.284 47.244) (width 0.5) (layer "F.Cu") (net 8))
 (segment (start 113.284 47.244) (end 113.792 46.736) (width 0.5) (layer "F.Cu") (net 8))
 (via (at 113.792 46.736) (size 1) (drill 0.5) (layers "F.Cu" "B.Cu") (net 8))
 (segment (start 169.418 103.632) (end 169.418 102.87) (width 0.5) (layer "B.Cu") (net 8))
 (segment (start 146.558 73.352) (end 146.558 48.768) (width 0.5) (layer "B.Cu") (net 8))
 (segment (start 147.32 103.378) (end 152.654 103.378) (width 0.5) (layer "B.Cu") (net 8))
 (segment (start 155.956 106.934) (end 166.116 106.934) (width 0.5) (layer "B.Cu") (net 8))
 (segment (start 146.304 77.724) (end 146.304 102.362) (width 0.5) (layer "B.Cu") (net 8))
 (segment (start 148.617 75.411) (end 146.558 73.352) (width 0.5) (layer "B.Cu") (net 8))
 (segment (start 152.654 103.378) (end 152.654 103.632) (width 0.5) (layer "B.Cu") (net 8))
 (segment (start 146.304 102.362) (end 147.32 103.378) (width 0.5) (layer "B.Cu") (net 8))
 (segment (start 152.654 103.632) (end 155.956 106.934) (width 0.5) (layer "B.Cu") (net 8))
 (segment (start 144.526 46.736) (end 113.792 46.736) (width 0.5) (layer "B.Cu") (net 8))
 (segment (start 146.558 48.768) (end 144.526 46.736) (width 0.5) (layer "B.Cu") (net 8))
 (segment (start 109.23 53.838) (end 113.284 53.838) (width 0.5) (layer "B.Cu") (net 8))
 (segment (start 148.617 75.411) (end 146.304 77.724) (width 0.5) (layer "B.Cu") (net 8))
 (segment (start 100.584 62.484) (end 109.23 53.838) (width 0.5) (layer "B.Cu") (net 8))
 (segment (start 166.116 106.934) (end 169.418 103.632) (width 0.5) (layer "B.Cu") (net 8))
 (segment (start 141.224 66.538) (end 138.684 69.078) (width 0.5) (layer "B.Cu") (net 20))
 (segment (start 140.462 51.562) (end 141.224 52.324) (width 0.5) (layer "B.Cu") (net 20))
 (segment (start 106.006 51.562) (end 140.462 51.562) (width 0.5) (layer "B.Cu") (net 20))
 (segment (start 100.584 56.984) (end 106.006 51.562) (width 0.5) (layer "B.Cu") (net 20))
 (segment (start 141.224 52.324) (end 141.224 66.538) (width 0.5) (layer "B.Cu") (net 20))
 (segment (start 134.366 48.514) (end 133.858 48.006) (width 0.2) (layer "F.Cu") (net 13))
 (segment (start 109.728 76.708) (end 109.728 48.26) (width 0.2) (layer "F.Cu") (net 13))
 (segment (start 134.366 82.54) (end 134.366 48.514) (width 0.2) (layer "F.Cu") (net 13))
 (segment (start 100.584 85.852) (end 109.728 76.708) (width 0.2) (layer "F.Cu") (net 13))
 (segment (start 138.684 86.858) (end 134.366 82.54) (width 0.2) (layer "F.Cu") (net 13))
 (via (at 133.858 48.006) (size 1) (drill 0.5) (layers "F.Cu" "B.Cu") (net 13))
 (via (at 109.728 48.26) (size 1) (drill 0.5) (layers "F.Cu" "B.Cu") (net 13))
 (segment (start 133.858 48.006) (end 109.982 48.006) (width 0.2) (layer "B.Cu") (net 13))
 (segment (start 109.982 48.006) (end 109.728 48.26) (width 0.2) (layer "B.Cu") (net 13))
 (segment (start 132.842 93.218) (end 134.112 94.488) (width 0.2) (layer "F.Cu") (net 10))
 (segment (start 107.95 49.276) (end 107.442 49.784) (width 0.2) (layer "F.Cu") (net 10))
 (segment (start 132.08 49.276) (end 132.842 50.038) (width 0.2) (layer "F.Cu") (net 10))
 (segment (start 107.442 73.494) (end 100.584 80.352) (width 0.2) (layer "F.Cu") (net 10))
 (segment (start 134.112 94.488) (end 134.122 94.478) (width 0.2) (layer "F.Cu") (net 10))
 (segment (start 132.842 50.038) (end 132.842 93.218) (width 0.2) (layer "F.Cu") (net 10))
 (segment (start 134.122 94.478) (end 138.684 94.478) (width 0.2) (layer "F.Cu") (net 10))
 (segment (start 107.442 49.784) (end 107.442 73.494) (width 0.2) (layer "F.Cu") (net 10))
 (via (at 107.95 49.276) (size 1) (drill 0.5) (layers "F.Cu" "B.Cu") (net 10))
 (via (at 132.08 49.276) (size 1) (drill 0.5) (layers "F.Cu" "B.Cu") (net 10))
 (segment (start 107.95 49.276) (end 132.08 49.276) (width 0.2) (layer "B.Cu") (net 10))
 (segment (start 95.25 50.292) (end 100.076 50.292) (width 0.2) (layer "F.Cu") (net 14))
 (segment (start 93.98 51.562) (end 95.25 50.292) (width 0.2) (layer "F.Cu") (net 14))
 (segment (start 100.584 74.852) (end 93.98 68.248) (width 0.2) (layer "F.Cu") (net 14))
 (segment (start 136.154 81.788) (end 136.144 81.788) (width 0.2) (layer "F.Cu") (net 14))
 (segment (start 136.144 50.8) (end 135.636 50.292) (width 0.2) (layer "F.Cu") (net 14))
 (segment (start 138.684 84.318) (end 136.154 81.788) (width 0.2) (layer "F.Cu") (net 14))
 (segment (start 136.144 81.788) (end 136.144 50.8) (width 0.2) (layer "F.Cu") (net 14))
 (segment (start 93.98 68.248) (end 93.98 51.562) (width 0.2) (layer "F.Cu") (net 14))
 (via (at 100.076 50.292) (size 1) (drill 0.5) (layers "F.Cu" "B.Cu") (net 14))
 (via (at 135.636 50.292) (size 1) (drill 0.5) (layers "F.Cu" "B.Cu") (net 14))
 (segment (start 135.636 50.292) (end 100.076 50.292) (width 0.2) (layer "B.Cu") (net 14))
 (segment (start 70.104 93.345) (end 68.072 91.313) (width 0.5) (layer "F.Cu") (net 1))
 (segment (start 78.74 93.345) (end 70.104 93.345) (width 0.5) (layer "F.Cu") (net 1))
 (segment (start 80.772 91.313) (end 78.74 93.345) (width 0.5) (layer "F.Cu") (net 1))
 (segment (start 82.804 62.357) (end 85.725 65.278) (width 0.5) (layer "B.Cu") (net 1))
 (segment (start 85.725 86.36) (end 80.772 91.313) (width 0.5) (layer "B.Cu") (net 1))
 (segment (start 85.725 65.278) (end 85.725 86.36) (width 0.5) (layer "B.Cu") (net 1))
 (segment (start 68.072 91.313) (end 68.072 84.709) (width 0.5) (layer "B.Cu") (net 1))
 (segment (start 138.684 81.778) (end 147.591 72.871) (width 0.2) (layer "F.Cu") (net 15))
 (segment (start 147.591 72.871) (end 148.617 72.871) (width 0.2) (layer "F.Cu") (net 15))
 (segment (start 167.386 100.584) (end 172.212 100.584) (width 0.2) (layer "F.Cu") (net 22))
 (segment (start 166.624 60.452) (end 166.624 99.822) (width 0.2) (layer "F.Cu") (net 22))
 (segment (start 138.684 63.998) (end 142.738 59.944) (width 0.2) (layer "F.Cu") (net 22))
 (segment (start 172.212 100.584) (end 174.498 102.87) (width 0.2) (layer "F.Cu") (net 22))
 (segment (start 166.624 99.822) (end 167.386 100.584) (width 0.2) (layer "F.Cu") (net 22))
 (segment (start 166.116 59.944) (end 166.624 60.452) (width 0.2) (layer "F.Cu") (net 22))
 (segment (start 142.738 59.944) (end 166.116 59.944) (width 0.2) (layer "F.Cu") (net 22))
 (segment (start 111.252 64.506) (end 111.252 44.45) (width 0.5) (layer "F.Cu") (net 31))
 (segment (start 111.252 44.45) (end 113.03 42.672) (width 0.5) (layer "F.Cu") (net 31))
 (segment (start 111.252 64.506) (end 113.284 66.538) (width 0.5) (layer "F.Cu") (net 31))
 (via (at 113.03 42.672) (size 1) (drill 0.5) (layers "F.Cu" "B.Cu") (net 31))
 (segment (start 161.798 92.71) (end 171.958 102.87) (width 0.5) (layer "B.Cu") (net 31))
 (segment (start 151.765 90.805) (end 153.67 92.71) (width 0.5) (layer "B.Cu") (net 31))
 (segment (start 149.987 42.672) (end 151.765 44.45) (width 0.5) (layer "B.Cu") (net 31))
 (segment (start 151.765 44.45) (end 151.765 90.805) (width 0.5) (layer "B.Cu") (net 31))
 (segment (start 153.67 92.71) (end 161.798 92.71) (width 0.5) (layer "B.Cu") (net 31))
 (segment (start 113.03 42.672) (end 149.987 42.672) (width 0.5) (layer "B.Cu") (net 31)))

